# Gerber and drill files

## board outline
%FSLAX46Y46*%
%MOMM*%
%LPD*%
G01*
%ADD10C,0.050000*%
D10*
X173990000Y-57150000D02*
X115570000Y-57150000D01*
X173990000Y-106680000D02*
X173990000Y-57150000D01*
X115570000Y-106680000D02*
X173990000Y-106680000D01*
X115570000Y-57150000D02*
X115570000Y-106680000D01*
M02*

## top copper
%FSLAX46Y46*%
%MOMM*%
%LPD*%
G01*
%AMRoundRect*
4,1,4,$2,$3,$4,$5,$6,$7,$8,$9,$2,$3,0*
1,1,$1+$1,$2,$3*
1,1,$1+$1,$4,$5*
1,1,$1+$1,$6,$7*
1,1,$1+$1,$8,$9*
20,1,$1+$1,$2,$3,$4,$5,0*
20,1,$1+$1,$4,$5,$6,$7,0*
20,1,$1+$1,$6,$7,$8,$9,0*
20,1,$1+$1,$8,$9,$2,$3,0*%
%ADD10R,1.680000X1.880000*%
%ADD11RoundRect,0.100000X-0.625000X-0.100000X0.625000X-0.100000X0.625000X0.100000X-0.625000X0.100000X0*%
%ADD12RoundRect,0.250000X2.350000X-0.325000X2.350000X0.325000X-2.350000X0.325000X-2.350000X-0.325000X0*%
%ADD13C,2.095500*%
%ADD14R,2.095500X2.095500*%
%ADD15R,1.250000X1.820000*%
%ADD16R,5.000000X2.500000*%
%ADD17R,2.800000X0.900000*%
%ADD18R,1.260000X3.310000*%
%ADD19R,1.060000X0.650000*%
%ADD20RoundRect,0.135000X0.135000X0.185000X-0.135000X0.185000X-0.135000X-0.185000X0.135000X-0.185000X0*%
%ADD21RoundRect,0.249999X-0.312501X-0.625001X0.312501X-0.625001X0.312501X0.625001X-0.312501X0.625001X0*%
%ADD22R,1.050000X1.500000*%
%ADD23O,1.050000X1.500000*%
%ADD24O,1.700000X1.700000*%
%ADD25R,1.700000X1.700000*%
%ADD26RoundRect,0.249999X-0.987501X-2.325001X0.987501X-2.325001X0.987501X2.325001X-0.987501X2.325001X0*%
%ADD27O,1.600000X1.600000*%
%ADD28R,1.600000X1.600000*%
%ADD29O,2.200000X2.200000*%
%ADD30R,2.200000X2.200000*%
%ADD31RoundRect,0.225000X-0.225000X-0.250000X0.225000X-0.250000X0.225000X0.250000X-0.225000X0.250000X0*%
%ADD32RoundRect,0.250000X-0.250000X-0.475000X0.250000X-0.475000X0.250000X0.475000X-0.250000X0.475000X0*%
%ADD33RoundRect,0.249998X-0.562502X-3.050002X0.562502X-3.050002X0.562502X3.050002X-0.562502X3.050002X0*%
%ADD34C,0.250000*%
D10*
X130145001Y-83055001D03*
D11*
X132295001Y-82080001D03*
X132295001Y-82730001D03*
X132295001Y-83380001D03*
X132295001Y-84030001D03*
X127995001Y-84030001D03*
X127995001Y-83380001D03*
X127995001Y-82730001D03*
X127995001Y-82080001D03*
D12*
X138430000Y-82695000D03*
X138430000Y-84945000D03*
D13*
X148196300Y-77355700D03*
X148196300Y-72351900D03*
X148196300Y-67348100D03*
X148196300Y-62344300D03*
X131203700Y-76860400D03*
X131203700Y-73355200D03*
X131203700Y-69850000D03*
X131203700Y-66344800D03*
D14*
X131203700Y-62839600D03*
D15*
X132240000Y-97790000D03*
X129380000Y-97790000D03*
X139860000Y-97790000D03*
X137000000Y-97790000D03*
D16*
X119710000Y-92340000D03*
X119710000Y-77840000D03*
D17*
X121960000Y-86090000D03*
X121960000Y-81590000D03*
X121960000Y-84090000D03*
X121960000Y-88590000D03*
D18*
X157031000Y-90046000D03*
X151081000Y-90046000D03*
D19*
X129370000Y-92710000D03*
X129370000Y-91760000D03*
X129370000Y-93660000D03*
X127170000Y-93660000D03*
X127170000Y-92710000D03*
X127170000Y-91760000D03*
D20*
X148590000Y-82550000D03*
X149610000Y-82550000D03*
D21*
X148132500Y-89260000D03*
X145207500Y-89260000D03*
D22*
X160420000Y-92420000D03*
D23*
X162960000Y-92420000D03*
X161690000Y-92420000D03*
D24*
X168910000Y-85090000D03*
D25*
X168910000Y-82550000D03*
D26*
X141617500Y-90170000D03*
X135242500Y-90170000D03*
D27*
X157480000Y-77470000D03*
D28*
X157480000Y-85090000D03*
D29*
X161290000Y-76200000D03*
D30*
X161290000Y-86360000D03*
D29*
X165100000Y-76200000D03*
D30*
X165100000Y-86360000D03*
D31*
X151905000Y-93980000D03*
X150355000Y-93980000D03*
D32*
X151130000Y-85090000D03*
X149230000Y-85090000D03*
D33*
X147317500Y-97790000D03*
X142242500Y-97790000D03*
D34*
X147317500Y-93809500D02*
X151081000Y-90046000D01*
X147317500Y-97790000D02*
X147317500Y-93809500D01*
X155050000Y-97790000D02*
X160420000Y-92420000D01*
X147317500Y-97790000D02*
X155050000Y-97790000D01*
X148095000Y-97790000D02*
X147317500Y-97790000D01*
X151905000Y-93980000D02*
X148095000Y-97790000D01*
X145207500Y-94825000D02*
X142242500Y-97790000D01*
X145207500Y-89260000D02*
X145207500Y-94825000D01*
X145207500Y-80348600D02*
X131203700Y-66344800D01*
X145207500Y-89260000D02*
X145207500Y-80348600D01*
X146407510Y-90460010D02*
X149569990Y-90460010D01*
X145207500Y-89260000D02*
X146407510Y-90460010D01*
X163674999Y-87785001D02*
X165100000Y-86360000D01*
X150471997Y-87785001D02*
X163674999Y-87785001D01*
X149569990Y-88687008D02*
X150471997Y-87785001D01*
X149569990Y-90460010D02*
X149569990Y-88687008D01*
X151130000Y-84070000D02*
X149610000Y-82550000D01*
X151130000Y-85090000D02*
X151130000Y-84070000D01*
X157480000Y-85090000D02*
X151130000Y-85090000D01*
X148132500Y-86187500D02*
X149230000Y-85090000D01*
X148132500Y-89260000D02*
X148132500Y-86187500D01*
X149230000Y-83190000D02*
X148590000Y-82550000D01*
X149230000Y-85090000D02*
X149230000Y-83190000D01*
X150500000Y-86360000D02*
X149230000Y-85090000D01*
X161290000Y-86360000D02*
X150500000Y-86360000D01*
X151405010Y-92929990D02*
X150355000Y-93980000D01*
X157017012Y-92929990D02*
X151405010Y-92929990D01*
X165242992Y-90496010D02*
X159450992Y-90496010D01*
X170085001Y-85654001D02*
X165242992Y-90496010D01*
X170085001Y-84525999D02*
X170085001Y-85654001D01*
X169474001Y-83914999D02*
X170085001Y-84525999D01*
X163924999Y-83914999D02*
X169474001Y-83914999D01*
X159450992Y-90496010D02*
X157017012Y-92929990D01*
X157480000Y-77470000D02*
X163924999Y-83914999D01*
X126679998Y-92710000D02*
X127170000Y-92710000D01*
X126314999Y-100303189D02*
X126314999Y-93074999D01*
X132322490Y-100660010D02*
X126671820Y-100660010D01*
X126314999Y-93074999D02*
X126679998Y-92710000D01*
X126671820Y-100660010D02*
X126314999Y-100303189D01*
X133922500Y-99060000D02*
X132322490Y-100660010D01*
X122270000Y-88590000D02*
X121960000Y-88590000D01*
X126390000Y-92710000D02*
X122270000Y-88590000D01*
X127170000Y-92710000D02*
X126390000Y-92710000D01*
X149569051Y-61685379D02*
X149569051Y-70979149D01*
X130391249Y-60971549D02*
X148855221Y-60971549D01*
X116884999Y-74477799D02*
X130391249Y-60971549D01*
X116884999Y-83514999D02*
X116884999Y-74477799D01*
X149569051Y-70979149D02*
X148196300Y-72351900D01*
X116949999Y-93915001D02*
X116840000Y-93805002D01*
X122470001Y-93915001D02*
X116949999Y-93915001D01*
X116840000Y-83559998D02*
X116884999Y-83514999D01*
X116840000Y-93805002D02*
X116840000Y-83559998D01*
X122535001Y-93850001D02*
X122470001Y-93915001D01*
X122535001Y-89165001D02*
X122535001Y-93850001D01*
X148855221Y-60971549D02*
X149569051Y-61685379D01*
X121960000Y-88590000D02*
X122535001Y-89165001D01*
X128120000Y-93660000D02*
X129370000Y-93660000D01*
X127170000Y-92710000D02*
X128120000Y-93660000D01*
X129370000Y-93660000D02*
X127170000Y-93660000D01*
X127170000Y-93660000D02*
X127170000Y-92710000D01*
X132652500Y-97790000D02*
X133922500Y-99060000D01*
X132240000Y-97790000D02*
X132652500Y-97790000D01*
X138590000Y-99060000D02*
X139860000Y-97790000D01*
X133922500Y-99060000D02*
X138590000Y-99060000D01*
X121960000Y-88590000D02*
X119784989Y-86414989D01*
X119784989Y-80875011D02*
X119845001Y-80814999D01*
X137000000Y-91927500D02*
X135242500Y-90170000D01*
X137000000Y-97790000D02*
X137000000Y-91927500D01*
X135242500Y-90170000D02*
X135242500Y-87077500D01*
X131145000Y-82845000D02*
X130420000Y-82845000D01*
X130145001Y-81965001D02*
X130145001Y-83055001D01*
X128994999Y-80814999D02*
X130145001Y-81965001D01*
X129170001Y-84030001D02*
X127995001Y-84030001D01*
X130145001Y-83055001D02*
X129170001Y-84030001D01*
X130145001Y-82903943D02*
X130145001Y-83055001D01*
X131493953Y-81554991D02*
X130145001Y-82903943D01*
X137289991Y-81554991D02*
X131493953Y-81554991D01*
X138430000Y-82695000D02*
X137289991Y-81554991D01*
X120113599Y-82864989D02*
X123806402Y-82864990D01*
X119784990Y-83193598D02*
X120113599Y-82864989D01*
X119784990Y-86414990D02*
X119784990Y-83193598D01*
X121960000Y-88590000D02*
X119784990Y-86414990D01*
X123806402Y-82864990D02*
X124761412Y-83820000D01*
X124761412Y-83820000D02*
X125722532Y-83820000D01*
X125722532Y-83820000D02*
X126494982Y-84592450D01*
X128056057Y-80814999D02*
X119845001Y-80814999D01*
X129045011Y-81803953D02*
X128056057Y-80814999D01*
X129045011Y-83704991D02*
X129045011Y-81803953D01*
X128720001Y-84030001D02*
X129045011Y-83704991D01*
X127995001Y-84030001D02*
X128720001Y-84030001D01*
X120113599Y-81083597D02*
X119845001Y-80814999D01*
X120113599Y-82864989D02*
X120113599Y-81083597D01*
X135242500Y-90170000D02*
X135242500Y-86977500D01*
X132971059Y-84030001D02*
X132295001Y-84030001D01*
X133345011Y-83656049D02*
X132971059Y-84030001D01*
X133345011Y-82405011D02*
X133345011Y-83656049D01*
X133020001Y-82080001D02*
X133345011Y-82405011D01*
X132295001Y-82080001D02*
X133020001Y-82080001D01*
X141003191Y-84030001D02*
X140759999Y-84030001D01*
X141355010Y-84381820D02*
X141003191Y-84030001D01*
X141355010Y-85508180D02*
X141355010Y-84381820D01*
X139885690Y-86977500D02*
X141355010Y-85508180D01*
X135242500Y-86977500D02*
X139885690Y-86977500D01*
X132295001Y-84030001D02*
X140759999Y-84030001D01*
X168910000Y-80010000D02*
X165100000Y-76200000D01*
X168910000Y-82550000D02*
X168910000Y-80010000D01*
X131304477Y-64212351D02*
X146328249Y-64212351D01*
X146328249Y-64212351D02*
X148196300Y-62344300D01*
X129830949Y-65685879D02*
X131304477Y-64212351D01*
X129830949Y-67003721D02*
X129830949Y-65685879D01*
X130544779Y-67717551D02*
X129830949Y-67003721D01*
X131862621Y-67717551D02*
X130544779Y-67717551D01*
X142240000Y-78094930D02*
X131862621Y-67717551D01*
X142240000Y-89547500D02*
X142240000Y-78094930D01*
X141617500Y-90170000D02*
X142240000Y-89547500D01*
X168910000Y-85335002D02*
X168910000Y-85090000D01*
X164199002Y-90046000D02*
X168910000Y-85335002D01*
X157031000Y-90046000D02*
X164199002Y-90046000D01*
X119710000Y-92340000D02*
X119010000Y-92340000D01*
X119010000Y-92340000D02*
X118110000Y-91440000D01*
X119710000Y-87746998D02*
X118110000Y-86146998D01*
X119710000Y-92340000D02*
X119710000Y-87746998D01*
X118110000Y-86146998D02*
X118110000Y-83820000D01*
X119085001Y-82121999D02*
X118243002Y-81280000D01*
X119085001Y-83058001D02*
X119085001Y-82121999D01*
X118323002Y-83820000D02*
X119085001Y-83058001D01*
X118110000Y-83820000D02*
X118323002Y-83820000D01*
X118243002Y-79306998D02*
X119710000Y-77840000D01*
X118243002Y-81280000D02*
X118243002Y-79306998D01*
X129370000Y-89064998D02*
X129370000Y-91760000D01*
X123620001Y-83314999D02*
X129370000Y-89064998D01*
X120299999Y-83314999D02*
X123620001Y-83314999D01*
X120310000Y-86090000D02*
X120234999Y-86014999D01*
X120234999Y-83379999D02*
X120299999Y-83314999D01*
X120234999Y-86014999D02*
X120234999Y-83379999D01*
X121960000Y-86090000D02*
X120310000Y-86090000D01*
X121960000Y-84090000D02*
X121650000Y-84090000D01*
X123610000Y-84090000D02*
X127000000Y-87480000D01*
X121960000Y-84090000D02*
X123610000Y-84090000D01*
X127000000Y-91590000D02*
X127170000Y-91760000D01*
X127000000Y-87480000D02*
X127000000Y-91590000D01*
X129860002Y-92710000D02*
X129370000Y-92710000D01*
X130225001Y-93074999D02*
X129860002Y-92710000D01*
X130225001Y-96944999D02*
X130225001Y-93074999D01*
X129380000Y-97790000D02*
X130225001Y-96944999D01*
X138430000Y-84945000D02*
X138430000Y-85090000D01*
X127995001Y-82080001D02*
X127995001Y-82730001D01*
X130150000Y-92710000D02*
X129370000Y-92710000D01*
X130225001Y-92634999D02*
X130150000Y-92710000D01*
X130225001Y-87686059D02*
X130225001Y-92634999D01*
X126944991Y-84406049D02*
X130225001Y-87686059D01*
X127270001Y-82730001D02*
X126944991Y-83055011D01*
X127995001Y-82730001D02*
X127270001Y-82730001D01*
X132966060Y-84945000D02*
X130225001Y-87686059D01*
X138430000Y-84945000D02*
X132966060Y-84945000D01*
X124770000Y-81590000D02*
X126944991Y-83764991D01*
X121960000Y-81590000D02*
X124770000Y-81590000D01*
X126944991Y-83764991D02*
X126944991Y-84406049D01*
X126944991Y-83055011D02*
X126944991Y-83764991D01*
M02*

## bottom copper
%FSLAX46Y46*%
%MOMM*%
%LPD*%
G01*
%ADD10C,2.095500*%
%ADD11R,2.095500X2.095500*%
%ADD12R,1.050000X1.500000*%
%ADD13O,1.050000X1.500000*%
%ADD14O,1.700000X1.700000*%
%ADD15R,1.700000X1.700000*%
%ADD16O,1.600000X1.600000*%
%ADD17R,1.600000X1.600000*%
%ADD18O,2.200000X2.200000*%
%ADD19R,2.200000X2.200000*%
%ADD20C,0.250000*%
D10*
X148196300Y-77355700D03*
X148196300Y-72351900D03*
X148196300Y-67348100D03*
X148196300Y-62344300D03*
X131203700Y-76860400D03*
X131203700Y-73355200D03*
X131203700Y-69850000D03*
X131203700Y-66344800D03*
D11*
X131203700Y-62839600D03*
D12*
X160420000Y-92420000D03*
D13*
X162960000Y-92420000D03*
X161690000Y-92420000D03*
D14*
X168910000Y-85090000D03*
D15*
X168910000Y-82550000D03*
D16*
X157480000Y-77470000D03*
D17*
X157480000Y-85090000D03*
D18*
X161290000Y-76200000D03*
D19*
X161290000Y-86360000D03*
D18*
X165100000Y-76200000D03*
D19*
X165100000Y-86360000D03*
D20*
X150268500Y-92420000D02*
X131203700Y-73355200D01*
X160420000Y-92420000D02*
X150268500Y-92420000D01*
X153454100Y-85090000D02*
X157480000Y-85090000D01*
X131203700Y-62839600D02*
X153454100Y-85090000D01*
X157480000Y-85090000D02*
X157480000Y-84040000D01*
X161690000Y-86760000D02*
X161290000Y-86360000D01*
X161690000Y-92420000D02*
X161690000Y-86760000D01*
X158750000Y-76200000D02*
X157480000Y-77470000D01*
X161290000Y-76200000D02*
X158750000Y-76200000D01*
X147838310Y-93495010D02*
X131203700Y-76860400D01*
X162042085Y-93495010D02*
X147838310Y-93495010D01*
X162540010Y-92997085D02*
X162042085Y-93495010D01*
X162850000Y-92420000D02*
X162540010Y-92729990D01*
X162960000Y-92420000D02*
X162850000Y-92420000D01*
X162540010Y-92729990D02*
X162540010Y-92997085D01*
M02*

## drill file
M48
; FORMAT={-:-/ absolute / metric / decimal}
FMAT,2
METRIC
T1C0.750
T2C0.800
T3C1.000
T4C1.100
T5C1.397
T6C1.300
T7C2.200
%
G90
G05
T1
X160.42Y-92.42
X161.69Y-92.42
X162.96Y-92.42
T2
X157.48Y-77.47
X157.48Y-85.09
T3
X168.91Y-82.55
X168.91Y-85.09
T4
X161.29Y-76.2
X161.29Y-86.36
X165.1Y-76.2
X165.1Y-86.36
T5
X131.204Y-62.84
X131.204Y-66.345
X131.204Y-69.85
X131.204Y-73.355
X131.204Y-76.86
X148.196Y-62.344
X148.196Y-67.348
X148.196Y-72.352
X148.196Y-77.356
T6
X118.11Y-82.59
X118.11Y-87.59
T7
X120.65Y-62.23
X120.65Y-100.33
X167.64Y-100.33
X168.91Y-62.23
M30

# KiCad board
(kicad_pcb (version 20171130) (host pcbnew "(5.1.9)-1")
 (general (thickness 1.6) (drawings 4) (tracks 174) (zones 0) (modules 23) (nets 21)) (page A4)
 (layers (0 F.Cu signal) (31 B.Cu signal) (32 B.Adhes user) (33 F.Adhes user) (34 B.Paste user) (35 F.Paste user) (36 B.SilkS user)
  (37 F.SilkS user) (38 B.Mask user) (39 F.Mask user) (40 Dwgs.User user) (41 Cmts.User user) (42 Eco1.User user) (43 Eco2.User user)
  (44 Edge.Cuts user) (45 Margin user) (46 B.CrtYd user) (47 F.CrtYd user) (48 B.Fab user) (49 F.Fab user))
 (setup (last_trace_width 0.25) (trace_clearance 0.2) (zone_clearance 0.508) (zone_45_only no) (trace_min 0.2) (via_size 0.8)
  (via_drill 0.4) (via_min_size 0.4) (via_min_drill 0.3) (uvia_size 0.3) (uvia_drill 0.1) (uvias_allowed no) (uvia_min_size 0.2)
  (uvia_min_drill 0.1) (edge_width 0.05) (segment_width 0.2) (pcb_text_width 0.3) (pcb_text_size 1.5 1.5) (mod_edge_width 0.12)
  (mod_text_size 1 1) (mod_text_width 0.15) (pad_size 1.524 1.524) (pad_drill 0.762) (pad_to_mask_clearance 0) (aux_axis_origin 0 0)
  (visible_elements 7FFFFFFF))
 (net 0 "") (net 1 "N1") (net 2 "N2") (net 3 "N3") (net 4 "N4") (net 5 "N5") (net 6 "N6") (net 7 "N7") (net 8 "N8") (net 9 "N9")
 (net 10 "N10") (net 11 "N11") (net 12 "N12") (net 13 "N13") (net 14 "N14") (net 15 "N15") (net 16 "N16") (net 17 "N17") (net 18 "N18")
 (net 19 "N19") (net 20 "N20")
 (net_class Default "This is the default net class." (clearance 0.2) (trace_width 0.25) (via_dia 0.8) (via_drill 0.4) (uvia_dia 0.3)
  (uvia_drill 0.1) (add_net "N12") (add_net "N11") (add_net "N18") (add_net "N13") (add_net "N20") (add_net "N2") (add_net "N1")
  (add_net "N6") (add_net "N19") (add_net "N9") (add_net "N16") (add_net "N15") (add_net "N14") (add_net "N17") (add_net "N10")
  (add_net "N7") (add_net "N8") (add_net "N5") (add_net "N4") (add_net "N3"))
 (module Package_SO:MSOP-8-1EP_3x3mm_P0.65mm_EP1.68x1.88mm (layer F.Cu) (at 130.145001 83.055001)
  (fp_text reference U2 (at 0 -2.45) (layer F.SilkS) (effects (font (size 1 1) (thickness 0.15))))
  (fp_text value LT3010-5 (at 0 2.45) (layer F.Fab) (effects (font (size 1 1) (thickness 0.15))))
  (pad "" smd roundrect (at 0.42 0.47) (size 0.68 0.76) (layers F.Paste) (roundrect_rratio 0.25))
  (pad "" smd roundrect (at 0.42 -0.47) (size 0.68 0.76) (layers F.Paste) (roundrect_rratio 0.25))
  (pad "" smd roundrect (at -0.42 0.47) (size 0.68 0.76) (layers F.Paste) (roundrect_rratio 0.25))
  (pad "" smd roundrect (at -0.42 -0.47) (size 0.68 0.76) (layers F.Paste) (roundrect_rratio 0.25))
  (pad 9 smd rect (at 0 0) (size 1.68 1.88) (layers F.Cu F.Mask) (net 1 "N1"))
  (pad 8 smd roundrect (at 2.15 -0.975) (size 1.45 0.4) (layers F.Cu F.Paste F.Mask) (roundrect_rratio 0.25) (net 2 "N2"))
  (pad 7 smd roundrect (at 2.15 -0.325) (size 1.45 0.4) (layers F.Cu F.Paste F.Mask) (roundrect_rratio 0.25) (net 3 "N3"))
  (pad 6 smd roundrect (at 2.15 0.325) (size 1.45 0.4) (layers F.Cu F.Paste F.Mask) (roundrect_rratio 0.25) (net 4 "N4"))
  (pad 5 smd roundrect (at 2.15 0.975) (size 1.45 0.4) (layers F.Cu F.Paste F.Mask) (roundrect_rratio 0.25) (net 2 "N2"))
  (pad 4 smd roundrect (at -2.15 0.975) (size 1.45 0.4) (layers F.Cu F.Paste F.Mask) (roundrect_rratio 0.25) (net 1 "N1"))
  (pad 3 smd roundrect (at -2.15 0.325) (size 1.45 0.4) (layers F.Cu F.Paste F.Mask) (roundrect_rratio 0.25) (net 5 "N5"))
  (pad 2 smd roundrect (at -2.15 -0.325) (size 1.45 0.4) (layers F.Cu F.Paste F.Mask) (roundrect_rratio 0.25) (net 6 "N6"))
  (pad 1 smd roundrect (at -2.15 -0.975) (size 1.45 0.4) (layers F.Cu F.Paste F.Mask) (roundrect_rratio 0.25) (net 6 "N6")))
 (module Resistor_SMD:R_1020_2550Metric (layer F.Cu) (at 138.43 83.82 90)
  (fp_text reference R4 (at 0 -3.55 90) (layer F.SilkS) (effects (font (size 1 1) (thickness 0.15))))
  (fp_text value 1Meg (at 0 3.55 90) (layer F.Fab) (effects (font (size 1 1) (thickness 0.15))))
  (pad 2 smd roundrect (at 1.125 0 90) (size 1.15 5.2) (layers F.Cu F.Paste F.Mask) (roundrect_rratio 0.217391) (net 1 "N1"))
  (pad 1 smd roundrect (at -1.125 0 90) (size 1.15 5.2) (layers F.Cu F.Paste F.Mask) (roundrect_rratio 0.217391) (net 6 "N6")))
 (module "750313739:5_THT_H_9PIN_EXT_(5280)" (layer F.Cu) (at 139.7 69.85)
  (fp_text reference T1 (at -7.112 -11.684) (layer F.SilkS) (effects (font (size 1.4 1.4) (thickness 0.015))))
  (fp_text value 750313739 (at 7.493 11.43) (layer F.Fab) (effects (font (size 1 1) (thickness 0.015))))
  (pad 6 thru_hole circle (at 8.4963 7.5057) (size 2.0955 2.0955) (drill 1.397) (layers *.Cu *.Mask) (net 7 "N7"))
  (pad 7 thru_hole circle (at 8.4963 2.5019) (size 2.0955 2.0955) (drill 1.397) (layers *.Cu *.Mask) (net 1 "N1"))
  (pad 8 thru_hole circle (at 8.4963 -2.5019) (size 2.0955 2.0955) (drill 1.397) (layers *.Cu *.Mask) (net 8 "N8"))
  (pad 9 thru_hole circle (at 8.4963 -7.5057) (size 2.0955 2.0955) (drill 1.397) (layers *.Cu *.Mask) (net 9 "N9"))
  (pad 5 thru_hole circle (at -8.4963 7.0104) (size 2.0955 2.0955) (drill 1.397) (layers *.Cu *.Mask) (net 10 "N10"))
  (pad 4 thru_hole circle (at -8.4963 3.5052) (size 2.0955 2.0955) (drill 1.397) (layers *.Cu *.Mask) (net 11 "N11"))
  (pad 3 thru_hole circle (at -8.4963 0) (size 2.0955 2.0955) (drill 1.397) (layers *.Cu *.Mask))
  (pad 2 thru_hole circle (at -8.4963 -3.5052) (size 2.0955 2.0955) (drill 1.397) (layers *.Cu *.Mask) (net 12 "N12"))
  (pad 1 thru_hole rect (at -8.4963 -7.0104) (size 2.0955 2.0955) (drill 1.397) (layers *.Cu *.Mask) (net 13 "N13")))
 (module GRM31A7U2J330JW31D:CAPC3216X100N (layer F.Cu) (at 130.81 97.79)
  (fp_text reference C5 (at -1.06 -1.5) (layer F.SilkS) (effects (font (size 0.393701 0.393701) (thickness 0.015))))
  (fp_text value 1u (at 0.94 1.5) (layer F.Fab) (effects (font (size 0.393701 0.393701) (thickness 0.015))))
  (pad 2 smd rect (at 1.43 0) (size 1.25 1.82) (layers F.Cu F.Paste F.Mask) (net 1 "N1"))
  (pad 1 smd rect (at -1.43 0) (size 1.25 1.82) (layers F.Cu F.Paste F.Mask) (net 6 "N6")))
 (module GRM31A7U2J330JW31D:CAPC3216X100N (layer F.Cu) (at 138.43 97.79)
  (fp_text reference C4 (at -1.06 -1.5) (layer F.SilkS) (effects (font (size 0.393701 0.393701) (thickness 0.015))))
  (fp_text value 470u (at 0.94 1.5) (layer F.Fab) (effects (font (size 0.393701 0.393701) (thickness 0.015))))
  (pad 2 smd rect (at 1.43 0) (size 1.25 1.82) (layers F.Cu F.Paste F.Mask) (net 1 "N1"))
  (pad 1 smd rect (at -1.43 0) (size 1.25 1.82) (layers F.Cu F.Paste F.Mask) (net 2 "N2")))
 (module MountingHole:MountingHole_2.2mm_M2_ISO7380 (layer F.Cu) (at 120.65 62.23)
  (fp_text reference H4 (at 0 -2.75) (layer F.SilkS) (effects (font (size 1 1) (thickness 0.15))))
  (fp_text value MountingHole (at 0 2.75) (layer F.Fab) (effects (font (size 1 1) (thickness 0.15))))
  (pad 1 np_thru_hole circle (at 0 0) (size 2.2 2.2) (drill 2.2) (layers *.Cu *.Mask)))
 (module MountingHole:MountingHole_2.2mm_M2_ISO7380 (layer F.Cu) (at 167.64 100.33)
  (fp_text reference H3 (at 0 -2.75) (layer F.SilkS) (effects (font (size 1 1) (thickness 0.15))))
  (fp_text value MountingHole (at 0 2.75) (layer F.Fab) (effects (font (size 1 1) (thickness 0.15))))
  (pad 1 np_thru_hole circle (at 0 0) (size 2.2 2.2) (drill 2.2) (layers *.Cu *.Mask)))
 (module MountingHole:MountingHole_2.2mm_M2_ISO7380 (layer F.Cu) (at 120.65 100.33)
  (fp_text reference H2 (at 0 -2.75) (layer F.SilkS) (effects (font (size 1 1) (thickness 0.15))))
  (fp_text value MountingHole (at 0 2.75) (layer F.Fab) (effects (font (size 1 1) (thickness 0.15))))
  (pad 1 np_thru_hole circle (at 0 0) (size 2.2 2.2) (drill 2.2) (layers *.Cu *.Mask)))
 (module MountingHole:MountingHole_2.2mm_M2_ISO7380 (layer F.Cu) (at 168.91 62.23)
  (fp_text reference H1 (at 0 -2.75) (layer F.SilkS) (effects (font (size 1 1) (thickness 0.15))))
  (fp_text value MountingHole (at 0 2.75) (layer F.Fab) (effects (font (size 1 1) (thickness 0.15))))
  (pad 1 np_thru_hole circle (at 0 0) (size 2.2 2.2) (drill 2.2) (layers *.Cu *.Mask)))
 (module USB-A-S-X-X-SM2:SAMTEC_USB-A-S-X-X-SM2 (layer F.Cu) (at 118.11 85.09 270)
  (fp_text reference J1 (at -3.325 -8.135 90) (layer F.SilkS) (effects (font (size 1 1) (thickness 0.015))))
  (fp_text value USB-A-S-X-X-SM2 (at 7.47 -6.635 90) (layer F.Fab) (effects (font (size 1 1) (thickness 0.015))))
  (pad S2 smd rect (at 7.25 -1.6 270) (size 2.5 5) (layers F.Cu F.Paste F.Mask) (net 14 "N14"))
  (pad S1 smd rect (at -7.25 -1.6 270) (size 2.5 5) (layers F.Cu F.Paste F.Mask) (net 14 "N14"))
  (pad 03 smd rect (at 1 -3.85 270) (size 0.9 2.8) (layers F.Cu F.Paste F.Mask) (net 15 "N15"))
  (pad 01 smd rect (at -3.5 -3.85 270) (size 0.9 2.8) (layers F.Cu F.Paste F.Mask) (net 6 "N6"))
  (pad 02 smd rect (at -1 -3.85 270) (size 0.9 2.8) (layers F.Cu F.Paste F.Mask) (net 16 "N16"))
  (pad 04 smd rect (at 3.5 -3.85 270) (size 0.9 2.8) (layers F.Cu F.Paste F.Mask) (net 1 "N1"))
  (pad None np_thru_hole circle (at 2.5 0 270) (size 1.3 1.3) (drill 1.3) (layers *.Cu *.Mask))
  (pad None np_thru_hole circle (at -2.5 0 270) (size 1.3 1.3) (drill 1.3) (layers *.Cu *.Mask)))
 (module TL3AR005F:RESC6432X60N (layer F.Cu) (at 154.056 90.046)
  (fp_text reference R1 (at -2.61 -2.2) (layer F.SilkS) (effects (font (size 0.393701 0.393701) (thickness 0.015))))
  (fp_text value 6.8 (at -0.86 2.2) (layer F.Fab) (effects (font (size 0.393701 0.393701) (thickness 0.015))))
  (pad 2 smd rect (at 2.975 0) (size 1.26 3.31) (layers F.Cu F.Paste F.Mask) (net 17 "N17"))
  (pad 1 smd rect (at -2.975 0) (size 1.26 3.31) (layers F.Cu F.Paste F.Mask) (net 11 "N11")))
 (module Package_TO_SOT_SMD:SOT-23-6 (layer F.Cu) (at 128.27 92.71)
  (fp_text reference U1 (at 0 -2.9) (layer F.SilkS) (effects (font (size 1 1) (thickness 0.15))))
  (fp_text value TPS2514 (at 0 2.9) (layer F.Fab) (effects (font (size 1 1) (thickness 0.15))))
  (pad 5 smd rect (at 1.1 0) (size 1.06 0.65) (layers F.Cu F.Paste F.Mask) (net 6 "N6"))
  (pad 6 smd rect (at 1.1 -0.95) (size 1.06 0.65) (layers F.Cu F.Paste F.Mask) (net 15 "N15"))
  (pad 4 smd rect (at 1.1 0.95) (size 1.06 0.65) (layers F.Cu F.Paste F.Mask) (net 1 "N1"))
  (pad 3 smd rect (at -1.1 0.95) (size 1.06 0.65) (layers F.Cu F.Paste F.Mask) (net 1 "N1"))
  (pad 2 smd rect (at -1.1 0) (size 1.06 0.65) (layers F.Cu F.Paste F.Mask) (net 1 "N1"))
  (pad 1 smd rect (at -1.1 -0.95) (size 1.06 0.65) (layers F.Cu F.Paste F.Mask) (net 16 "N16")))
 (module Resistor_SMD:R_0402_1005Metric (layer F.Cu) (at 149.1 82.55 180)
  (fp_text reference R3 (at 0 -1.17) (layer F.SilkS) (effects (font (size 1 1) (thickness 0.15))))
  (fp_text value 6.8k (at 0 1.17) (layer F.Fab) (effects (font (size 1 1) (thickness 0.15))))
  (pad 2 smd roundrect (at 0.51 0 180) (size 0.54 0.64) (layers F.Cu F.Paste F.Mask) (roundrect_rratio 0.25) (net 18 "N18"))
  (pad 1 smd roundrect (at -0.51 0 180) (size 0.54 0.64) (layers F.Cu F.Paste F.Mask) (roundrect_rratio 0.25) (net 13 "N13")))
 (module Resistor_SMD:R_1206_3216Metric (layer F.Cu) (at 146.67 89.26)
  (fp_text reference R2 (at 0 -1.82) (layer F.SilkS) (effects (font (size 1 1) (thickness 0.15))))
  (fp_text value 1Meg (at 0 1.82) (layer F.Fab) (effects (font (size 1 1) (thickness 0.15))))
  (pad 2 smd roundrect (at 1.4625 0) (size 1.125 1.75) (layers F.Cu F.Paste F.Mask) (roundrect_rratio 0.2222213333333333) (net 18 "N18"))
  (pad 1 smd roundrect (at -1.4625 0) (size 1.125 1.75) (layers F.Cu F.Paste F.Mask) (roundrect_rratio 0.2222213333333333) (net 12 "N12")))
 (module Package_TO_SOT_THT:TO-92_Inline (layer F.Cu) (at 160.42 92.42)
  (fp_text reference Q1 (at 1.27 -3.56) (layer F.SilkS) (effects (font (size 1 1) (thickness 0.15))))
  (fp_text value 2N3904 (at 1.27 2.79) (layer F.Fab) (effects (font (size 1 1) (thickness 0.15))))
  (pad 1 thru_hole rect (at 0 0) (size 1.05 1.5) (drill 0.75) (layers *.Cu *.Mask) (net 11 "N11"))
  (pad 3 thru_hole oval (at 2.54 0) (size 1.05 1.5) (drill 0.75) (layers *.Cu *.Mask) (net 10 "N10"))
  (pad 2 thru_hole oval (at 1.27 0) (size 1.05 1.5) (drill 0.75) (layers *.Cu *.Mask) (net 18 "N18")))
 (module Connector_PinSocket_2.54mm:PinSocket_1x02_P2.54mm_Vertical (layer F.Cu) (at 168.91 82.55)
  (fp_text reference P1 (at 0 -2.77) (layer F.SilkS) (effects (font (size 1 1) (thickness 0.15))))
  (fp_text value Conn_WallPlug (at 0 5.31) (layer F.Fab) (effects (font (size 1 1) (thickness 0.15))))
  (pad 2 thru_hole oval (at 0 2.54) (size 1.7 1.7) (drill 1) (layers *.Cu *.Mask) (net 17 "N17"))
  (pad 1 thru_hole rect (at 0 0) (size 1.7 1.7) (drill 1) (layers *.Cu *.Mask) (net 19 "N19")))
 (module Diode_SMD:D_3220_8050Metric (layer F.Cu) (at 138.43 90.17)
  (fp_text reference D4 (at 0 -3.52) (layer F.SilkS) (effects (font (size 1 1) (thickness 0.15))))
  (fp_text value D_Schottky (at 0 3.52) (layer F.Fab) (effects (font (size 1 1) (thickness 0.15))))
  (pad 2 smd roundrect (at 3.1875 0) (size 2.475 5.15) (layers F.Cu F.Paste F.Mask) (roundrect_rratio 0.101009696969697) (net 9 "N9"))
  (pad 1 smd roundrect (at -3.1875 0) (size 2.475 5.15) (layers F.Cu F.Paste F.Mask) (roundrect_rratio 0.101009696969697) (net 2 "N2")))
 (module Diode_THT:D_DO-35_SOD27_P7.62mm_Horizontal (layer F.Cu) (at 157.48 85.09 90)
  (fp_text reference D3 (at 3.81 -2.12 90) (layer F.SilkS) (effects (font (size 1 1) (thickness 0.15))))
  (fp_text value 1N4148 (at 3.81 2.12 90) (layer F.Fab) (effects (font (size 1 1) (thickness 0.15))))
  (pad 2 thru_hole oval (at 7.62 0 90) (size 1.6 1.6) (drill 0.8) (layers *.Cu *.Mask) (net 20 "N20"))
  (pad 1 thru_hole rect (at 0 0 90) (size 1.6 1.6) (drill 0.8) (layers *.Cu *.Mask) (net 13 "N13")))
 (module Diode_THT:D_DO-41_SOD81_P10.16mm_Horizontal (layer F.Cu) (at 161.29 86.36 90)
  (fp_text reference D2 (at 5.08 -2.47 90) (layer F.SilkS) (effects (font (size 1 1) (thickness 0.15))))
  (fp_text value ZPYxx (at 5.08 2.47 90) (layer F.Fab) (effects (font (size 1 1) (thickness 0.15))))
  (pad 2 thru_hole oval (at 10.16 0 90) (size 2.2 2.2) (drill 1.1) (layers *.Cu *.Mask) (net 20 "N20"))
  (pad 1 thru_hole rect (at 0 0 90) (size 2.2 2.2) (drill 1.1) (layers *.Cu *.Mask) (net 18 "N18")))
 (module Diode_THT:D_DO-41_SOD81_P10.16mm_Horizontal (layer F.Cu) (at 165.1 86.36 90)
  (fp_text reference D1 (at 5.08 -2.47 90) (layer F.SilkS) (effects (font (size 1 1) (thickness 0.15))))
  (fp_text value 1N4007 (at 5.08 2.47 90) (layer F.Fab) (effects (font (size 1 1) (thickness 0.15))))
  (pad 2 thru_hole oval (at 10.16 0 90) (size 2.2 2.2) (drill 1.1) (layers *.Cu *.Mask) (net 19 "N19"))
  (pad 1 thru_hole rect (at 0 0 90) (size 2.2 2.2) (drill 1.1) (layers *.Cu *.Mask) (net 12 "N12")))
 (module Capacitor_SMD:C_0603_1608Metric (layer F.Cu) (at 151.13 93.98)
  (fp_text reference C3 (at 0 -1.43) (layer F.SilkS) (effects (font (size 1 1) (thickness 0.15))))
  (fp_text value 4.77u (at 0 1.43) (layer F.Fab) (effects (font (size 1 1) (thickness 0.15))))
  (pad 2 smd roundrect (at 0.775 0) (size 0.9 0.95) (layers F.Cu F.Paste F.Mask) (roundrect_rratio 0.25) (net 11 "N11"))
  (pad 1 smd roundrect (at -0.775 0) (size 0.9 0.95) (layers F.Cu F.Paste F.Mask) (roundrect_rratio 0.25) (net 20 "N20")))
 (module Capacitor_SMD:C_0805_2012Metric (layer F.Cu) (at 150.18 85.09)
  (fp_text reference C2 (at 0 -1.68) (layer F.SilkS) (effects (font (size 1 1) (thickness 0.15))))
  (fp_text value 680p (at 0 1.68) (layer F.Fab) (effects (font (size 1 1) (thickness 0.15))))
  (pad 2 smd roundrect (at 0.95 0) (size 1 1.45) (layers F.Cu F.Paste F.Mask) (roundrect_rratio 0.25) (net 13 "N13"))
  (pad 1 smd roundrect (at -0.95 0) (size 1 1.45) (layers F.Cu F.Paste F.Mask) (roundrect_rratio 0.25) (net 18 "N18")))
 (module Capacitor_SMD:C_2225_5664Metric (layer F.Cu) (at 144.78 97.79)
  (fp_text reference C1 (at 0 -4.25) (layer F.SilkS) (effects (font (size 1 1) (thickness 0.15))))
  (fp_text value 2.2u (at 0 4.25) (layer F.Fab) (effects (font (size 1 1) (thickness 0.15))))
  (pad 2 smd roundrect (at 2.5375 0) (size 1.625 6.6) (layers F.Cu F.Paste F.Mask) (roundrect_rratio 0.1538449230769231) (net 11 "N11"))
  (pad 1 smd roundrect (at -2.5375 0) (size 1.625 6.6) (layers F.Cu F.Paste F.Mask) (roundrect_rratio 0.1538449230769231) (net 12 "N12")))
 (gr_line (start 173.99 57.15) (end 115.57 57.15) (layer Edge.Cuts) (width 0.05))
 (gr_line (start 173.99 106.68) (end 173.99 57.15) (layer Edge.Cuts) (width 0.05))
 (gr_line (start 115.57 106.68) (end 173.99 106.68) (layer Edge.Cuts) (width 0.05))
 (gr_line (start 115.57 57.15) (end 115.57 106.68) (layer Edge.Cuts) (width 0.05))
 (segment (start 147.3175 93.8095) (end 151.081 90.046) (width 0.25) (layer F.Cu) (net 11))
 (segment (start 147.3175 97.79) (end 147.3175 93.8095) (width 0.25) (layer F.Cu) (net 11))
 (segment (start 155.05 97.79) (end 160.42 92.42) (width 0.25) (layer F.Cu) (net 11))
 (segment (start 147.3175 97.79) (end 155.05 97.79) (width 0.25) (layer F.Cu) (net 11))
 (segment (start 148.095 97.79) (end 147.3175 97.79) (width 0.25) (layer F.Cu) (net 11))
 (segment (start 151.905 93.98) (end 148.095 97.79) (width 0.25) (layer F.Cu) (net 11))
 (segment (start 150.2685 92.42) (end 131.2037 73.3552) (width 0.25) (layer B.Cu) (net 11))
 (segment (start 160.42 92.42) (end 150.2685 92.42) (width 0.25) (layer B.Cu) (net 11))
 (segment (start 145.2075 94.825) (end 142.2425 97.79) (width 0.25) (layer F.Cu) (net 12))
 (segment (start 145.2075 89.26) (end 145.2075 94.825) (width 0.25) (layer F.Cu) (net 12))
 (segment (start 145.2075 80.3486) (end 131.2037 66.3448) (width 0.25) (layer F.Cu) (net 12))
 (segment (start 145.2075 89.26) (end 145.2075 80.3486) (width 0.25) (layer F.Cu) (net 12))
 (segment (start 146.40751 90.46001) (end 149.56999 90.46001) (width 0.25) (layer F.Cu) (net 12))
 (segment (start 145.2075 89.26) (end 146.40751 90.46001) (width 0.25) (layer F.Cu) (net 12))
 (segment (start 163.674999 87.785001) (end 165.1 86.36) (width 0.25) (layer F.Cu) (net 12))
 (segment (start 150.471997 87.785001) (end 163.674999 87.785001) (width 0.25) (layer F.Cu) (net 12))
 (segment (start 149.56999 88.687008) (end 150.471997 87.785001) (width 0.25) (layer F.Cu) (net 12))
 (segment (start 149.56999 90.46001) (end 149.56999 88.687008) (width 0.25) (layer F.Cu) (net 12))
 (segment (start 153.4541 85.09) (end 157.48 85.09) (width 0.25) (layer B.Cu) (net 13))
 (segment (start 131.2037 62.8396) (end 153.4541 85.09) (width 0.25) (layer B.Cu) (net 13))
 (segment (start 157.48 85.09) (end 157.48 84.04) (width 0.25) (layer B.Cu) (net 13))
 (segment (start 151.13 84.07) (end 149.61 82.55) (width 0.25) (layer F.Cu) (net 13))
 (segment (start 151.13 85.09) (end 151.13 84.07) (width 0.25) (layer F.Cu) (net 13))
 (segment (start 157.48 85.09) (end 151.13 85.09) (width 0.25) (layer F.Cu) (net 13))
 (segment (start 161.69 86.76) (end 161.29 86.36) (width 0.25) (layer B.Cu) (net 18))
 (segment (start 161.69 92.42) (end 161.69 86.76) (width 0.25) (layer B.Cu) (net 18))
 (segment (start 148.1325 86.1875) (end 149.23 85.09) (width 0.25) (layer F.Cu) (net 18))
 (segment (start 148.1325 89.26) (end 148.1325 86.1875) (width 0.25) (layer F.Cu) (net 18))
 (segment (start 149.23 83.19) (end 148.59 82.55) (width 0.25) (layer F.Cu) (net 18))
 (segment (start 149.23 85.09) (end 149.23 83.19) (width 0.25) (layer F.Cu) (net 18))
 (segment (start 150.5 86.36) (end 149.23 85.09) (width 0.25) (layer F.Cu) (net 18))
 (segment (start 161.29 86.36) (end 150.5 86.36) (width 0.25) (layer F.Cu) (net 18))
 (segment (start 158.75 76.2) (end 157.48 77.47) (width 0.25) (layer B.Cu) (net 20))
 (segment (start 161.29 76.2) (end 158.75 76.2) (width 0.25) (layer B.Cu) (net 20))
 (segment (start 151.40501 92.92999) (end 150.355 93.98) (width 0.25) (layer F.Cu) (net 20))
 (segment (start 157.017012 92.92999) (end 151.40501 92.92999) (width 0.25) (layer F.Cu) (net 20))
 (segment (start 165.242992 90.49601) (end 159.450992 90.49601) (width 0.25) (layer F.Cu) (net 20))
 (segment (start 170.085001 85.654001) (end 165.242992 90.49601) (width 0.25) (layer F.Cu) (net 20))
 (segment (start 170.085001 84.525999) (end 170.085001 85.654001) (width 0.25) (layer F.Cu) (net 20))
 (segment (start 169.474001 83.914999) (end 170.085001 84.525999) (width 0.25) (layer F.Cu) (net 20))
 (segment (start 163.924999 83.914999) (end 169.474001 83.914999) (width 0.25) (layer F.Cu) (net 20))
 (segment (start 159.450992 90.49601) (end 157.017012 92.92999) (width 0.25) (layer F.Cu) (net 20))
 (segment (start 157.48 77.47) (end 163.924999 83.914999) (width 0.25) (layer F.Cu) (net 20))
 (segment (start 126.679998 92.71) (end 127.17 92.71) (width 0.25) (layer F.Cu) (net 1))
 (segment (start 126.314999 100.303189) (end 126.314999 93.074999) (width 0.25) (layer F.Cu) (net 1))
 (segment (start 132.32249 100.66001) (end 126.67182 100.66001) (width 0.25) (layer F.Cu) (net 1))
 (segment (start 126.314999 93.074999) (end 126.679998 92.71) (width 0.25) (layer F.Cu) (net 1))
 (segment (start 126.67182 100.66001) (end 126.314999 100.303189) (width 0.25) (layer F.Cu) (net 1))
 (segment (start 133.9225 99.06) (end 132.32249 100.66001) (width 0.25) (layer F.Cu) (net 1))
 (segment (start 122.27 88.59) (end 121.96 88.59) (width 0.25) (layer F.Cu) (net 1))
 (segment (start 126.39 92.71) (end 122.27 88.59) (width 0.25) (layer F.Cu) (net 1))
 (segment (start 127.17 92.71) (end 126.39 92.71) (width 0.25) (layer F.Cu) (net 1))
 (segment (start 149.569051 61.685379) (end 149.569051 70.979149) (width 0.25) (layer F.Cu) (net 1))
 (segment (start 130.391249 60.971549) (end 148.855221 60.971549) (width 0.25) (layer F.Cu) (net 1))
 (segment (start 116.884999 74.477799) (end 130.391249 60.971549) (width 0.25) (layer F.Cu) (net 1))
 (segment (start 116.884999 83.514999) (end 116.884999 74.477799) (width 0.25) (layer F.Cu) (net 1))
 (segment (start 149.569051 70.979149) (end 148.1963 72.3519) (width 0.25) (layer F.Cu) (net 1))
 (segment (start 116.949999 93.915001) (end 116.84 93.805002) (width 0.25) (layer F.Cu) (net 1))
 (segment (start 122.470001 93.915001) (end 116.949999 93.915001) (width 0.25) (layer F.Cu) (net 1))
 (segment (start 116.84 83.559998) (end 116.884999 83.514999) (width 0.25) (layer F.Cu) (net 1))
 (segment (start 116.84 93.805002) (end 116.84 83.559998) (width 0.25) (layer F.Cu) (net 1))
 (segment (start 122.535001 93.850001) (end 122.470001 93.915001) (width 0.25) (layer F.Cu) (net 1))
 (segment (start 122.535001 89.165001) (end 122.535001 93.850001) (width 0.25) (layer F.Cu) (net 1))
 (segment (start 148.855221 60.971549) (end 149.569051 61.685379) (width 0.25) (layer F.Cu) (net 1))
 (segment (start 121.96 88.59) (end 122.535001 89.165001) (width 0.25) (layer F.Cu) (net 1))
 (segment (start 128.12 93.66) (end 129.37 93.66) (width 0.25) (layer F.Cu) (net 1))
 (segment (start 127.17 92.71) (end 128.12 93.66) (width 0.25) (layer F.Cu) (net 1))
 (segment (start 129.37 93.66) (end 127.17 93.66) (width 0.25) (layer F.Cu) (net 1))
 (segment (start 127.17 93.66) (end 127.17 92.71) (width 0.25) (layer F.Cu) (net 1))
 (segment (start 132.6525 97.79) (end 133.9225 99.06) (width 0.25) (layer F.Cu) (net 1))
 (segment (start 132.24 97.79) (end 132.6525 97.79) (width 0.25) (layer F.Cu) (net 1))
 (segment (start 138.59 99.06) (end 139.86 97.79) (width 0.25) (layer F.Cu) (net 1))
 (segment (start 133.9225 99.06) (end 138.59 99.06) (width 0.25) (layer F.Cu) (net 1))
 (segment (start 121.96 88.59) (end 119.784989 86.414989) (width 0.25) (layer F.Cu) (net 1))
 (segment (start 119.784989 80.875011) (end 119.845001 80.814999) (width 0.25) (layer F.Cu) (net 1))
 (segment (start 137 91.9275) (end 135.2425 90.17) (width 0.25) (layer F.Cu) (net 2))
 (segment (start 137 97.79) (end 137 91.9275) (width 0.25) (layer F.Cu) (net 2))
 (segment (start 135.2425 90.17) (end 135.2425 87.0775) (width 0.25) (layer F.Cu) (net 2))
 (segment (start 131.145 82.845) (end 130.42 82.845) (width 0.25) (layer F.Cu) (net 1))
 (segment (start 130.145001 81.965001) (end 130.145001 83.055001) (width 0.25) (layer F.Cu) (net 1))
 (segment (start 128.994999 80.814999) (end 130.145001 81.965001) (width 0.25) (layer F.Cu) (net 1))
 (segment (start 129.170001 84.030001) (end 127.995001 84.030001) (width 0.25) (layer F.Cu) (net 1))
 (segment (start 130.145001 83.055001) (end 129.170001 84.030001) (width 0.25) (layer F.Cu) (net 1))
 (segment (start 130.145001 82.903943) (end 130.145001 83.055001) (width 0.25) (layer F.Cu) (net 1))
 (segment (start 131.493953 81.554991) (end 130.145001 82.903943) (width 0.25) (layer F.Cu) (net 1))
 (segment (start 137.289991 81.554991) (end 131.493953 81.554991) (width 0.25) (layer F.Cu) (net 1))
 (segment (start 138.43 82.695) (end 137.289991 81.554991) (width 0.25) (layer F.Cu) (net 1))
 (segment (start 120.113599 82.864989) (end 123.806402 82.86499) (width 0.25) (layer F.Cu) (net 1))
 (segment (start 119.78499 83.193598) (end 120.113599 82.864989) (width 0.25) (layer F.Cu) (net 1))
 (segment (start 119.78499 86.41499) (end 119.78499 83.193598) (width 0.25) (layer F.Cu) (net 1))
 (segment (start 121.96 88.59) (end 119.78499 86.41499) (width 0.25) (layer F.Cu) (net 1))
 (segment (start 123.806402 82.86499) (end 124.761412 83.82) (width 0.25) (layer F.Cu) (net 1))
 (segment (start 124.761412 83.82) (end 125.722532 83.82) (width 0.25) (layer F.Cu) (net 1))
 (segment (start 125.722532 83.82) (end 126.494982 84.59245) (width 0.25) (layer F.Cu) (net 1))
 (segment (start 128.056057 80.814999) (end 119.845001 80.814999) (width 0.25) (layer F.Cu) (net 1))
 (segment (start 129.045011 81.803953) (end 128.056057 80.814999) (width 0.25) (layer F.Cu) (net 1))
 (segment (start 129.045011 83.704991) (end 129.045011 81.803953) (width 0.25) (layer F.Cu) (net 1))
 (segment (start 128.720001 84.030001) (end 129.045011 83.704991) (width 0.25) (layer F.Cu) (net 1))
 (segment (start 127.995001 84.030001) (end 128.720001 84.030001) (width 0.25) (layer F.Cu) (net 1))
 (segment (start 120.113599 81.083597) (end 119.845001 80.814999) (width 0.25) (layer F.Cu) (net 1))
 (segment (start 120.113599 82.864989) (end 120.113599 81.083597) (width 0.25) (layer F.Cu) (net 1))
 (segment (start 135.2425 90.17) (end 135.2425 86.9775) (width 0.25) (layer F.Cu) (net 2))
 (segment (start 132.971059 84.030001) (end 132.295001 84.030001) (width 0.25) (layer F.Cu) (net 2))
 (segment (start 133.345011 83.656049) (end 132.971059 84.030001) (width 0.25) (layer F.Cu) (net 2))
 (segment (start 133.345011 82.405011) (end 133.345011 83.656049) (width 0.25) (layer F.Cu) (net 2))
 (segment (start 133.020001 82.080001) (end 133.345011 82.405011) (width 0.25) (layer F.Cu) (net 2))
 (segment (start 132.295001 82.080001) (end 133.020001 82.080001) (width 0.25) (layer F.Cu) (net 2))
 (segment (start 141.003191 84.030001) (end 140.759999 84.030001) (width 0.25) (layer F.Cu) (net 2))
 (segment (start 141.35501 84.38182) (end 141.003191 84.030001) (width 0.25) (layer F.Cu) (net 2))
 (segment (start 141.35501 85.50818) (end 141.35501 84.38182) (width 0.25) (layer F.Cu) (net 2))
 (segment (start 139.88569 86.9775) (end 141.35501 85.50818) (width 0.25) (layer F.Cu) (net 2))
 (segment (start 135.2425 86.9775) (end 139.88569 86.9775) (width 0.25) (layer F.Cu) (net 2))
 (segment (start 132.295001 84.030001) (end 140.759999 84.030001) (width 0.25) (layer F.Cu) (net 2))
 (segment (start 168.91 80.01) (end 165.1 76.2) (width 0.25) (layer F.Cu) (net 19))
 (segment (start 168.91 82.55) (end 168.91 80.01) (width 0.25) (layer F.Cu) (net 19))
 (segment (start 131.304477 64.212351) (end 146.328249 64.212351) (width 0.25) (layer F.Cu) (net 9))
 (segment (start 146.328249 64.212351) (end 148.1963 62.3443) (width 0.25) (layer F.Cu) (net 9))
 (segment (start 129.830949 65.685879) (end 131.304477 64.212351) (width 0.25) (layer F.Cu) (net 9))
 (segment (start 129.830949 67.003721) (end 129.830949 65.685879) (width 0.25) (layer F.Cu) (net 9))
 (segment (start 130.544779 67.717551) (end 129.830949 67.003721) (width 0.25) (layer F.Cu) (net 9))
 (segment (start 131.862621 67.717551) (end 130.544779 67.717551) (width 0.25) (layer F.Cu) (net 9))
 (segment (start 142.24 78.09493) (end 131.862621 67.717551) (width 0.25) (layer F.Cu) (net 9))
 (segment (start 142.24 89.5475) (end 142.24 78.09493) (width 0.25) (layer F.Cu) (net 9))
 (segment (start 141.6175 90.17) (end 142.24 89.5475) (width 0.25) (layer F.Cu) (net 9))
 (segment (start 168.91 85.335002) (end 168.91 85.09) (width 0.25) (layer F.Cu) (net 17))
 (segment (start 164.199002 90.046) (end 168.91 85.335002) (width 0.25) (layer F.Cu) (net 17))
 (segment (start 157.031 90.046) (end 164.199002 90.046) (width 0.25) (layer F.Cu) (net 17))
 (segment (start 147.83831 93.49501) (end 131.2037 76.8604) (width 0.25) (layer B.Cu) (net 10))
 (segment (start 162.042085 93.49501) (end 147.83831 93.49501) (width 0.25) (layer B.Cu) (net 10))
 (segment (start 162.54001 92.997085) (end 162.042085 93.49501) (width 0.25) (layer B.Cu) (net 10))
 (segment (start 162.85 92.42) (end 162.54001 92.72999) (width 0.25) (layer B.Cu) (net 10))
 (segment (start 162.96 92.42) (end 162.85 92.42) (width 0.25) (layer B.Cu) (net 10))
 (segment (start 162.54001 92.72999) (end 162.54001 92.997085) (width 0.25) (layer B.Cu) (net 10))
 (segment (start 119.71 92.34) (end 119.01 92.34) (width 0.25) (layer F.Cu) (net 14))
 (segment (start 119.01 92.34) (end 118.11 91.44) (width 0.25) (layer F.Cu) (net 14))
 (segment (start 119.71 87.746998) (end 118.11 86.146998) (width 0.25) (layer F.Cu) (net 14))
 (segment (start 119.71 92.34) (end 119.71 87.746998) (width 0.25) (layer F.Cu) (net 14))
 (segment (start 118.11 86.146998) (end 118.11 83.82) (width 0.25) (layer F.Cu) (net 14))
 (segment (start 119.085001 82.121999) (end 118.243002 81.28) (width 0.25) (layer F.Cu) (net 14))
 (segment (start 119.085001 83.058001) (end 119.085001 82.121999) (width 0.25) (layer F.Cu) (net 14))
 (segment (start 118.323002 83.82) (end 119.085001 83.058001) (width 0.25) (layer F.Cu) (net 14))
 (segment (start 118.11 83.82) (end 118.323002 83.82) (width 0.25) (layer F.Cu) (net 14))
 (segment (start 118.243002 79.306998) (end 119.71 77.84) (width 0.25) (layer F.Cu) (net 14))
 (segment (start 118.243002 81.28) (end 118.243002 79.306998) (width 0.25) (layer F.Cu) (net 14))
 (segment (start 129.37 89.064998) (end 129.37 91.76) (width 0.25) (layer F.Cu) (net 15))
 (segment (start 123.620001 83.314999) (end 129.37 89.064998) (width 0.25) (layer F.Cu) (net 15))
 (segment (start 120.299999 83.314999) (end 123.620001 83.314999) (width 0.25) (layer F.Cu) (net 15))
 (segment (start 120.31 86.09) (end 120.234999 86.014999) (width 0.25) (layer F.Cu) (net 15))
 (segment (start 120.234999 83.379999) (end 120.299999 83.314999) (width 0.25) (layer F.Cu) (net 15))
 (segment (start 120.234999 86.014999) (end 120.234999 83.379999) (width 0.25) (layer F.Cu) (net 15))
 (segment (start 121.96 86.09) (end 120.31 86.09) (width 0.25) (layer F.Cu) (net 15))
 (segment (start 121.96 84.09) (end 121.65 84.09) (width 0.25) (layer F.Cu) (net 16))
 (segment (start 123.61 84.09) (end 127 87.48) (width 0.25) (layer F.Cu) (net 16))
 (segment (start 121.96 84.09) (end 123.61 84.09) (width 0.25) (layer F.Cu) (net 16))
 (segment (start 127 91.59) (end 127.17 91.76) (width 0.25) (layer F.Cu) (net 16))
 (segment (start 127 87.48) (end 127 91.59) (width 0.25) (layer F.Cu) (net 16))
 (segment (start 129.860002 92.71) (end 129.37 92.71) (width 0.25) (layer F.Cu) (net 6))
 (segment (start 130.225001 93.074999) (end 129.860002 92.71) (width 0.25) (layer F.Cu) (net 6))
 (segment (start 130.225001 96.944999) (end 130.225001 93.074999) (width 0.25) (layer F.Cu) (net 6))
 (segment (start 129.38 97.79) (end 130.225001 96.944999) (width 0.25) (layer F.Cu) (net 6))
 (segment (start 138.43 84.945) (end 138.43 85.09) (width 0.25) (layer F.Cu) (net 6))
 (segment (start 127.995001 82.080001) (end 127.995001 82.730001) (width 0.25) (layer F.Cu) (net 6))
 (segment (start 130.15 92.71) (end 129.37 92.71) (width 0.25) (layer F.Cu) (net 6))
 (segment (start 130.225001 92.634999) (end 130.15 92.71) (width 0.25) (layer F.Cu) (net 6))
 (segment (start 130.225001 87.686059) (end 130.225001 92.634999) (width 0.25) (layer F.Cu) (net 6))
 (segment (start 126.944991 84.406049) (end 130.225001 87.686059) (width 0.25) (layer F.Cu) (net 6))
 (segment (start 127.270001 82.730001) (end 126.944991 83.055011) (width 0.25) (layer F.Cu) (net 6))
 (segment (start 127.995001 82.730001) (end 127.270001 82.730001) (width 0.25) (layer F.Cu) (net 6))
 (segment (start 132.96606 84.945) (end 130.225001 87.686059) (width 0.25) (layer F.Cu) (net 6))
 (segment (start 138.43 84.945) (end 132.96606 84.945) (width 0.25) (layer F.Cu) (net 6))
 (segment (start 124.77 81.59) (end 126.944991 83.764991) (width 0.25) (layer F.Cu) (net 6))
 (segment (start 121.96 81.59) (end 124.77 81.59) (width 0.25) (layer F.Cu) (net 6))
 (segment (start 126.944991 83.764991) (end 126.944991 84.406049) (width 0.25) (layer F.Cu) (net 6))
 (segment (start 126.944991 83.055011) (end 126.944991 83.764991) (width 0.25) (layer F.Cu) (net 6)))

